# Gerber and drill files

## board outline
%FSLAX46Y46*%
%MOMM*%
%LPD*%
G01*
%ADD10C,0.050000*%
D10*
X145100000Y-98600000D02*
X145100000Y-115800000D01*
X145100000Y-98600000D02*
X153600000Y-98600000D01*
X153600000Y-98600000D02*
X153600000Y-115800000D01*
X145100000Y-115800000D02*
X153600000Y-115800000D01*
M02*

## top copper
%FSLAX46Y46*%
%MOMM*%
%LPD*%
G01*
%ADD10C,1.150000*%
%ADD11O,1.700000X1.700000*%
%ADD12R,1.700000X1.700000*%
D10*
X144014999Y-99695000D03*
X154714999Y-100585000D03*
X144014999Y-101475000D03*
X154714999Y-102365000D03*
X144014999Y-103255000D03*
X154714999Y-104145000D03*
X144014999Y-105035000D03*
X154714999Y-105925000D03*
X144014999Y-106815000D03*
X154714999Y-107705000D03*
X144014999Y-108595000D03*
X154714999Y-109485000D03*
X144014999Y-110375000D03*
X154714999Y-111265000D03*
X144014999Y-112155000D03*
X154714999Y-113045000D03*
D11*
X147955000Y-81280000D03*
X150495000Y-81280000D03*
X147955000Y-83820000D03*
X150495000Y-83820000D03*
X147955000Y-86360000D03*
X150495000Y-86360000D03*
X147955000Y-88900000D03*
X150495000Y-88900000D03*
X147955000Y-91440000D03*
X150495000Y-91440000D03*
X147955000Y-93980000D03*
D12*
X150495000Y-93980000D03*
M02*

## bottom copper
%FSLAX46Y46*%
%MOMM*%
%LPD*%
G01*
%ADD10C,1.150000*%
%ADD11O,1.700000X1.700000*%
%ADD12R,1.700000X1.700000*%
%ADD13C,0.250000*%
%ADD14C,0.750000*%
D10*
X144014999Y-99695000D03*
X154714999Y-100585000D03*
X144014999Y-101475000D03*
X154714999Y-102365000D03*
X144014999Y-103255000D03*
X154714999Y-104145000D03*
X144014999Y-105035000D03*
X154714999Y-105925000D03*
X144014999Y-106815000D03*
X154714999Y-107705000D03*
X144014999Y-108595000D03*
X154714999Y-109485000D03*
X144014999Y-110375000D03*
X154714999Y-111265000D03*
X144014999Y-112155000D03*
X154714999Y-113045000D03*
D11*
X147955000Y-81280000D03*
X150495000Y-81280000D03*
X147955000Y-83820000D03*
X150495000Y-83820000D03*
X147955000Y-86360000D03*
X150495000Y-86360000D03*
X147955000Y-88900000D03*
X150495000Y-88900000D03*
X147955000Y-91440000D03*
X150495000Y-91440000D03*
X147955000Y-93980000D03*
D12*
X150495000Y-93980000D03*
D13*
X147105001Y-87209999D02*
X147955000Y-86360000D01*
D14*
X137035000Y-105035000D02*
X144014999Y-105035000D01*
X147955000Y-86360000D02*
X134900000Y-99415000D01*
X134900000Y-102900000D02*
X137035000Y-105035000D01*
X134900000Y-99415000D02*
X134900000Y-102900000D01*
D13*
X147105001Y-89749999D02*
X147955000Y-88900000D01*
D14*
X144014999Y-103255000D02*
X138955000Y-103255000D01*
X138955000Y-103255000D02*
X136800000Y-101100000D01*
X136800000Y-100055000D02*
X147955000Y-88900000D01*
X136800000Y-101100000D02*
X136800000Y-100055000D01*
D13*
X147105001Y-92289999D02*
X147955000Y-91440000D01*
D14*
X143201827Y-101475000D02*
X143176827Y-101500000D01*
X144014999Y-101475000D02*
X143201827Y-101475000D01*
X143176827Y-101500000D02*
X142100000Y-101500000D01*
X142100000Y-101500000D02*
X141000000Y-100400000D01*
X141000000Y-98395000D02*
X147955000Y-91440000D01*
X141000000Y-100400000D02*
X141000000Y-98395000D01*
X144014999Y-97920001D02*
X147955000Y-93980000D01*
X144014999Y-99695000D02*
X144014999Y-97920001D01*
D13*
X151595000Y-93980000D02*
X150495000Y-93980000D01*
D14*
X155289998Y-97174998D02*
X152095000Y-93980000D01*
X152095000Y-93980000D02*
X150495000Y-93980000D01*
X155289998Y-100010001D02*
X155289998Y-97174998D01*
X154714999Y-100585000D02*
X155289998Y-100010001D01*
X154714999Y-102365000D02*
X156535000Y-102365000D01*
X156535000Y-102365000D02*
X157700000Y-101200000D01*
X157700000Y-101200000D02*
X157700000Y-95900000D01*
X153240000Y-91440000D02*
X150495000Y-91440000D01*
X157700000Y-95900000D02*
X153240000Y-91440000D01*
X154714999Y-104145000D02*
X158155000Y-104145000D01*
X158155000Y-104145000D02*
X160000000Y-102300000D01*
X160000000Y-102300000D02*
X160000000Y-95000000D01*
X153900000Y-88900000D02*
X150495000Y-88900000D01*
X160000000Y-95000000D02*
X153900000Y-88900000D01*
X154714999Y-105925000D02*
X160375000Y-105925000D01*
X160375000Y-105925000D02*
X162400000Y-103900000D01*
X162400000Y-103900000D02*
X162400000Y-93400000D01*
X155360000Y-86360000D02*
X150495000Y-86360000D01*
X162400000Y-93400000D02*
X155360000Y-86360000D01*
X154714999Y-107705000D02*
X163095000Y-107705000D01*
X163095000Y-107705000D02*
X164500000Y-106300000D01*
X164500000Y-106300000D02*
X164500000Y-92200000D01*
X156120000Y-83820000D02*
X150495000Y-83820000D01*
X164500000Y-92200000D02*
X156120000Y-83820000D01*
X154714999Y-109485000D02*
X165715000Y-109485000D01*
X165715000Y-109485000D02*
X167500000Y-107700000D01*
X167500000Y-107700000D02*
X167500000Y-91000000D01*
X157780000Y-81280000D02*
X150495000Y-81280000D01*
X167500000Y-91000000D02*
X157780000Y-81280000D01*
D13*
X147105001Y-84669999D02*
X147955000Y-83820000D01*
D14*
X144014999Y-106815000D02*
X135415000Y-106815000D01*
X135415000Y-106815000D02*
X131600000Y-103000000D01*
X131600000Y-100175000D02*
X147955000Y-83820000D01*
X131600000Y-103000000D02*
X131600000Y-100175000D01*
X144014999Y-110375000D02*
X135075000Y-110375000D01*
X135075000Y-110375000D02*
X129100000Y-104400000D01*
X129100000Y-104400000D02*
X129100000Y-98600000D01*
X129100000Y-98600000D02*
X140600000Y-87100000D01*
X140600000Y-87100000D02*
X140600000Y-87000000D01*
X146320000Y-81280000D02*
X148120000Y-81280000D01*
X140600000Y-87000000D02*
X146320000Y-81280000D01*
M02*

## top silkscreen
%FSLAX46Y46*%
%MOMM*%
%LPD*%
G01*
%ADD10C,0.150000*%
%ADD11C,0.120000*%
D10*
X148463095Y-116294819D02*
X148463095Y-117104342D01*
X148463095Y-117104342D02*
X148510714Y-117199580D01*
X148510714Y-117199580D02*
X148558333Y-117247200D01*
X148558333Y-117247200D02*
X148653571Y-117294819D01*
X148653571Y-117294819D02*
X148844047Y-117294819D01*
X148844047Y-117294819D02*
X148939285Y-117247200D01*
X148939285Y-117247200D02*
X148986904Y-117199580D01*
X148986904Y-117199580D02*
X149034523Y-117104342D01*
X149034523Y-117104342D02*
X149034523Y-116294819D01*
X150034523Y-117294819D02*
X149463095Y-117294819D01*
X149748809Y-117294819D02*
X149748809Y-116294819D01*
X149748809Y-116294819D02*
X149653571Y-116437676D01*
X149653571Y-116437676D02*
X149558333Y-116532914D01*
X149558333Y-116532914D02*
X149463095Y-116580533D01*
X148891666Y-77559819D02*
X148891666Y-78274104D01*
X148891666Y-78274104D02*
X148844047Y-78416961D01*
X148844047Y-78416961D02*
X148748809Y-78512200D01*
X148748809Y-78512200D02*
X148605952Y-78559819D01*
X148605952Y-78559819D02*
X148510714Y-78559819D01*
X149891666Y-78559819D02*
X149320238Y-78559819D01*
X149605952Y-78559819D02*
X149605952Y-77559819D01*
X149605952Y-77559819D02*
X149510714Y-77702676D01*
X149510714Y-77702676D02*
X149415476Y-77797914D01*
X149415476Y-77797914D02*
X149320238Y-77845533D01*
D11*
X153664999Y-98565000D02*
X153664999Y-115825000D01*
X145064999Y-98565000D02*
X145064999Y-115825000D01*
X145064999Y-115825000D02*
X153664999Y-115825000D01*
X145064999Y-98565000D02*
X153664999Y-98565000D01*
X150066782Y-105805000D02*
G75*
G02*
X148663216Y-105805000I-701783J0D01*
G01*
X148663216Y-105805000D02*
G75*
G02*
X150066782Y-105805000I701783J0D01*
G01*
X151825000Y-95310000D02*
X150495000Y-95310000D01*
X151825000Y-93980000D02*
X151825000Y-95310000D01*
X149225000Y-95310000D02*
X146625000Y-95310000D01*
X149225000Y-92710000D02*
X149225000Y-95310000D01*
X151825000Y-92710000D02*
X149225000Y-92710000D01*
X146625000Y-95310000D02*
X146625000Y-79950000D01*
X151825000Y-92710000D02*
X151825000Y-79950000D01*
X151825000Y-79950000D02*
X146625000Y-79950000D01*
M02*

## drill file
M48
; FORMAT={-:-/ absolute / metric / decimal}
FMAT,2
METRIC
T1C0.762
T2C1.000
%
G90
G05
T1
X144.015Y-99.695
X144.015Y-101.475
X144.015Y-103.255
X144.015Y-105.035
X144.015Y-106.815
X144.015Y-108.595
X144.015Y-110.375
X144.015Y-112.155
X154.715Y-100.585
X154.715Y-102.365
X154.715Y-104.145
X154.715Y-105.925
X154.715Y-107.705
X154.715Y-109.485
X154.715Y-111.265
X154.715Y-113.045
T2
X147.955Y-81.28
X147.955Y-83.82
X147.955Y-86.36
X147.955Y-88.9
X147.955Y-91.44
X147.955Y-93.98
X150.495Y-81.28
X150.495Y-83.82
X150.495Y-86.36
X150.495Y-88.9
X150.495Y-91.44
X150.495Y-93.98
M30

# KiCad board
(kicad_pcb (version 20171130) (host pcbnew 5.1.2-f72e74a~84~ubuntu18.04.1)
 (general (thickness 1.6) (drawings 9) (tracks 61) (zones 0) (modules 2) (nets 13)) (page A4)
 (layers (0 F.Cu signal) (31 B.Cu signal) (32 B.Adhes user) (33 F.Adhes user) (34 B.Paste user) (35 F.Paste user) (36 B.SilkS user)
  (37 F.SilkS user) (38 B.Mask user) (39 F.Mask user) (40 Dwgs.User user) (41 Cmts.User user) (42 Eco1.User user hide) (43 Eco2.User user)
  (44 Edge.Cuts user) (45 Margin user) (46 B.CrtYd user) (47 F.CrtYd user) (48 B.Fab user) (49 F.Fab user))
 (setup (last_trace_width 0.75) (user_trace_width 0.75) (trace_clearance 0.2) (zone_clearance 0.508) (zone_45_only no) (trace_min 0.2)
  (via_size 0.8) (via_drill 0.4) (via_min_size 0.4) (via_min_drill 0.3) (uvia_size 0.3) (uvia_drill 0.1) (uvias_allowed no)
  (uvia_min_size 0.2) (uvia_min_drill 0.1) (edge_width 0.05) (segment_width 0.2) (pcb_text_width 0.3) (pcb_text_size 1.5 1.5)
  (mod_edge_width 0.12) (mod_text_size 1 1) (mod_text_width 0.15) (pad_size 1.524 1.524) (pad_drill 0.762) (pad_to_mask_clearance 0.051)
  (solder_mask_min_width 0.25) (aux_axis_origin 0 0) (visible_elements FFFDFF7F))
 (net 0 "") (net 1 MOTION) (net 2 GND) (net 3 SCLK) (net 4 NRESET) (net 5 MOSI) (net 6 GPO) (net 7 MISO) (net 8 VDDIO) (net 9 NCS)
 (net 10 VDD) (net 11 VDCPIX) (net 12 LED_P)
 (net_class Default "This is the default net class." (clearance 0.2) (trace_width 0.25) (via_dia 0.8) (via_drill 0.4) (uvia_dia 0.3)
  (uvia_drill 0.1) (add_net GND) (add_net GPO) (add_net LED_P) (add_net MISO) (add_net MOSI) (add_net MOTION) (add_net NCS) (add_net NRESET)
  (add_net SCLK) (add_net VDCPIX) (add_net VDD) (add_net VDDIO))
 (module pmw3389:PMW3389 (layer F.Cu) (at 149.364999 105.805)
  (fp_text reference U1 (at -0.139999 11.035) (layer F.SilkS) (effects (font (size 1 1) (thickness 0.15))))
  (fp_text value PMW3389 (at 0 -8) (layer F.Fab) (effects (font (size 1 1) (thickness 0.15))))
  (fp_line (start 4.3 -7.24) (end 4.3 10.02) (layer F.SilkS) (width 0.12))
  (fp_line (start -4.3 -7.24) (end -4.3 10.02) (layer F.SilkS) (width 0.12))
  (fp_line (start -4.3 10.02) (end 4.3 10.02) (layer F.SilkS) (width 0.12))
  (fp_line (start -4.3 -7.24) (end 4.3 -7.24) (layer F.SilkS) (width 0.12))
  (fp_circle (center 0 0) (end 0.7 -0.05) (layer F.SilkS) (width 0.12))
  (pad 9 thru_hole circle (at -5.35 -6.11) (size 1.15 1.15) (drill 0.762) (layers *.Cu *.Mask) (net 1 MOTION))
  (pad 8 thru_hole circle (at 5.35 -5.22) (size 1.15 1.15) (drill 0.762) (layers *.Cu *.Mask) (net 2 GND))
  (pad 10 thru_hole circle (at -5.35 -4.33) (size 1.15 1.15) (drill 0.762) (layers *.Cu *.Mask) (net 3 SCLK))
  (pad 7 thru_hole circle (at 5.35 -3.44) (size 1.15 1.15) (drill 0.762) (layers *.Cu *.Mask) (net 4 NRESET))
  (pad 11 thru_hole circle (at -5.35 -2.55) (size 1.15 1.15) (drill 0.762) (layers *.Cu *.Mask) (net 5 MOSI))
  (pad 6 thru_hole circle (at 5.35 -1.66) (size 1.15 1.15) (drill 0.762) (layers *.Cu *.Mask) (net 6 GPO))
  (pad 12 thru_hole circle (at -5.35 -0.77) (size 1.15 1.15) (drill 0.762) (layers *.Cu *.Mask) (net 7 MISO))
  (pad 5 thru_hole circle (at 5.35 0.12) (size 1.15 1.15) (drill 0.762) (layers *.Cu *.Mask) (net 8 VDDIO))
  (pad 13 thru_hole circle (at -5.35 1.01) (size 1.15 1.15) (drill 0.762) (layers *.Cu *.Mask) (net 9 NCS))
  (pad 4 thru_hole circle (at 5.35 1.9) (size 1.15 1.15) (drill 0.762) (layers *.Cu *.Mask) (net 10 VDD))
  (pad 14 thru_hole circle (at -5.35 2.79) (size 1.15 1.15) (drill 0.762) (layers *.Cu *.Mask))
  (pad 3 thru_hole circle (at 5.35 3.68) (size 1.15 1.15) (drill 0.762) (layers *.Cu *.Mask) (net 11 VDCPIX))
  (pad 15 thru_hole circle (at -5.35 4.57) (size 1.15 1.15) (drill 0.762) (layers *.Cu *.Mask) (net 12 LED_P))
  (pad 2 thru_hole circle (at 5.35 5.46) (size 1.15 1.15) (drill 0.762) (layers *.Cu *.Mask))
  (pad 16 thru_hole circle (at -5.35 6.35) (size 1.15 1.15) (drill 0.762) (layers *.Cu *.Mask))
  (pad 1 thru_hole circle (at 5.35 7.24) (size 1.15 1.15) (drill 0.762) (layers *.Cu *.Mask)))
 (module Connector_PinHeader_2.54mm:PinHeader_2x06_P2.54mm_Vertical (layer F.Cu) (at 150.495 93.98 180)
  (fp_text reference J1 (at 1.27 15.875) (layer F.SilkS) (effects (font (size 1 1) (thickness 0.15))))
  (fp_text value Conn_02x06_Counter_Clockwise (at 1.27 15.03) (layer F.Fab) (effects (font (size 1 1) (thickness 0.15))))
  (fp_line (start -1.33 -1.33) (end 0 -1.33) (layer F.SilkS) (width 0.12))
  (fp_line (start -1.33 0) (end -1.33 -1.33) (layer F.SilkS) (width 0.12))
  (fp_line (start 1.27 -1.33) (end 3.87 -1.33) (layer F.SilkS) (width 0.12))
  (fp_line (start 1.27 1.27) (end 1.27 -1.33) (layer F.SilkS) (width 0.12))
  (fp_line (start -1.33 1.27) (end 1.27 1.27) (layer F.SilkS) (width 0.12))
  (fp_line (start 3.87 -1.33) (end 3.87 14.03) (layer F.SilkS) (width 0.12))
  (fp_line (start -1.33 1.27) (end -1.33 14.03) (layer F.SilkS) (width 0.12))
  (fp_line (start -1.33 14.03) (end 3.87 14.03) (layer F.SilkS) (width 0.12))
  (pad 12 thru_hole oval (at 2.54 12.7 180) (size 1.7 1.7) (drill 1) (layers *.Cu *.Mask) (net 12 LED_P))
  (pad 11 thru_hole oval (at 0 12.7 180) (size 1.7 1.7) (drill 1) (layers *.Cu *.Mask) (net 11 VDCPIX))
  (pad 10 thru_hole oval (at 2.54 10.16 180) (size 1.7 1.7) (drill 1) (layers *.Cu *.Mask) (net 9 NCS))
  (pad 9 thru_hole oval (at 0 10.16 180) (size 1.7 1.7) (drill 1) (layers *.Cu *.Mask) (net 10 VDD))
  (pad 8 thru_hole oval (at 2.54 7.62 180) (size 1.7 1.7) (drill 1) (layers *.Cu *.Mask) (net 7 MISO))
  (pad 7 thru_hole oval (at 0 7.62 180) (size 1.7 1.7) (drill 1) (layers *.Cu *.Mask) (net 8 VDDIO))
  (pad 6 thru_hole oval (at 2.54 5.08 180) (size 1.7 1.7) (drill 1) (layers *.Cu *.Mask) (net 5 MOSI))
  (pad 5 thru_hole oval (at 0 5.08 180) (size 1.7 1.7) (drill 1) (layers *.Cu *.Mask) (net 6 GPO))
  (pad 4 thru_hole oval (at 2.54 2.54 180) (size 1.7 1.7) (drill 1) (layers *.Cu *.Mask) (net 3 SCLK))
  (pad 3 thru_hole oval (at 0 2.54 180) (size 1.7 1.7) (drill 1) (layers *.Cu *.Mask) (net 4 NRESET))
  (pad 2 thru_hole oval (at 2.54 0 180) (size 1.7 1.7) (drill 1) (layers *.Cu *.Mask) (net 1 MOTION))
  (pad 1 thru_hole rect (at 0 0 180) (size 1.7 1.7) (drill 1) (layers *.Cu *.Mask) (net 2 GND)))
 (gr_line (start 145.1 98.6) (end 145.1 115.8) (layer Edge.Cuts) (width 0.05))
 (gr_line (start 145.1 98.6) (end 153.6 98.6) (layer Edge.Cuts) (width 0.05))
 (gr_line (start 153.6 98.6) (end 153.6 115.8) (layer Edge.Cuts) (width 0.05))
 (gr_line (start 145.1 115.8) (end 153.6 115.8) (layer Edge.Cuts) (width 0.05))
 (segment (start 147.105001 87.209999) (end 147.955 86.36) (width 0.25) (layer B.Cu) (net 7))
 (segment (start 137.035 105.035) (end 144.014999 105.035) (width 0.75) (layer B.Cu) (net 7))
 (segment (start 147.955 86.36) (end 134.9 99.415) (width 0.75) (layer B.Cu) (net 7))
 (segment (start 134.9 102.9) (end 137.035 105.035) (width 0.75) (layer B.Cu) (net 7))
 (segment (start 134.9 99.415) (end 134.9 102.9) (width 0.75) (layer B.Cu) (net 7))
 (segment (start 147.105001 89.749999) (end 147.955 88.9) (width 0.25) (layer B.Cu) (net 5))
 (segment (start 144.014999 103.255) (end 138.955 103.255) (width 0.75) (layer B.Cu) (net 5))
 (segment (start 138.955 103.255) (end 136.8 101.1) (width 0.75) (layer B.Cu) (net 5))
 (segment (start 136.8 100.055) (end 147.955 88.9) (width 0.75) (layer B.Cu) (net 5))
 (segment (start 136.8 101.1) (end 136.8 100.055) (width 0.75) (layer B.Cu) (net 5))
 (segment (start 147.105001 92.289999) (end 147.955 91.44) (width 0.25) (layer B.Cu) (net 3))
 (segment (start 143.201827 101.475) (end 143.176827 101.5) (width 0.75) (layer B.Cu) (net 3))
 (segment (start 144.014999 101.475) (end 143.201827 101.475) (width 0.75) (layer B.Cu) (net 3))
 (segment (start 143.176827 101.5) (end 142.1 101.5) (width 0.75) (layer B.Cu) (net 3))
 (segment (start 142.1 101.5) (end 141 100.4) (width 0.75) (layer B.Cu) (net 3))
 (segment (start 141 98.395) (end 147.955 91.44) (width 0.75) (layer B.Cu) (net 3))
 (segment (start 141 100.4) (end 141 98.395) (width 0.75) (layer B.Cu) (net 3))
 (segment (start 144.014999 97.920001) (end 147.955 93.98) (width 0.75) (layer B.Cu) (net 1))
 (segment (start 144.014999 99.695) (end 144.014999 97.920001) (width 0.75) (layer B.Cu) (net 1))
 (segment (start 151.595 93.98) (end 150.495 93.98) (width 0.25) (layer B.Cu) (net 2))
 (segment (start 155.289998 97.174998) (end 152.095 93.98) (width 0.75) (layer B.Cu) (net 2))
 (segment (start 152.095 93.98) (end 150.495 93.98) (width 0.75) (layer B.Cu) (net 2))
 (segment (start 155.289998 100.010001) (end 155.289998 97.174998) (width 0.75) (layer B.Cu) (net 2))
 (segment (start 154.714999 100.585) (end 155.289998 100.010001) (width 0.75) (layer B.Cu) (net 2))
 (segment (start 154.714999 102.365) (end 156.535 102.365) (width 0.75) (layer B.Cu) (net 4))
 (segment (start 156.535 102.365) (end 157.7 101.2) (width 0.75) (layer B.Cu) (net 4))
 (segment (start 157.7 101.2) (end 157.7 95.9) (width 0.75) (layer B.Cu) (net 4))
 (segment (start 153.24 91.44) (end 150.495 91.44) (width 0.75) (layer B.Cu) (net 4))
 (segment (start 157.7 95.9) (end 153.24 91.44) (width 0.75) (layer B.Cu) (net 4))
 (segment (start 154.714999 104.145) (end 158.155 104.145) (width 0.75) (layer B.Cu) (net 6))
 (segment (start 158.155 104.145) (end 160 102.3) (width 0.75) (layer B.Cu) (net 6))
 (segment (start 160 102.3) (end 160 95) (width 0.75) (layer B.Cu) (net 6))
 (segment (start 153.9 88.9) (end 150.495 88.9) (width 0.75) (layer B.Cu) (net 6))
 (segment (start 160 95) (end 153.9 88.9) (width 0.75) (layer B.Cu) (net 6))
 (segment (start 154.714999 105.925) (end 160.375 105.925) (width 0.75) (layer B.Cu) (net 8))
 (segment (start 160.375 105.925) (end 162.4 103.9) (width 0.75) (layer B.Cu) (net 8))
 (segment (start 162.4 103.9) (end 162.4 93.4) (width 0.75) (layer B.Cu) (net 8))
 (segment (start 155.36 86.36) (end 150.495 86.36) (width 0.75) (layer B.Cu) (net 8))
 (segment (start 162.4 93.4) (end 155.36 86.36) (width 0.75) (layer B.Cu) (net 8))
 (segment (start 154.714999 107.705) (end 163.095 107.705) (width 0.75) (layer B.Cu) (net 10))
 (segment (start 163.095 107.705) (end 164.5 106.3) (width 0.75) (layer B.Cu) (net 10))
 (segment (start 164.5 106.3) (end 164.5 92.2) (width 0.75) (layer B.Cu) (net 10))
 (segment (start 156.12 83.82) (end 150.495 83.82) (width 0.75) (layer B.Cu) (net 10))
 (segment (start 164.5 92.2) (end 156.12 83.82) (width 0.75) (layer B.Cu) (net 10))
 (segment (start 154.714999 109.485) (end 165.715 109.485) (width 0.75) (layer B.Cu) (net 11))
 (segment (start 165.715 109.485) (end 167.5 107.7) (width 0.75) (layer B.Cu) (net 11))
 (segment (start 167.5 107.7) (end 167.5 91) (width 0.75) (layer B.Cu) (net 11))
 (segment (start 157.78 81.28) (end 150.495 81.28) (width 0.75) (layer B.Cu) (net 11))
 (segment (start 167.5 91) (end 157.78 81.28) (width 0.75) (layer B.Cu) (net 11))
 (segment (start 147.105001 84.669999) (end 147.955 83.82) (width 0.25) (layer B.Cu) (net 9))
 (segment (start 144.014999 106.815) (end 135.415 106.815) (width 0.75) (layer B.Cu) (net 9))
 (segment (start 135.415 106.815) (end 131.6 103) (width 0.75) (layer B.Cu) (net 9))
 (segment (start 131.6 100.175) (end 147.955 83.82) (width 0.75) (layer B.Cu) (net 9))
 (segment (start 131.6 103) (end 131.6 100.175) (width 0.75) (layer B.Cu) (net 9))
 (segment (start 144.014999 110.375) (end 135.075 110.375) (width 0.75) (layer B.Cu) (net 12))
 (segment (start 135.075 110.375) (end 129.1 104.4) (width 0.75) (layer B.Cu) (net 12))
 (segment (start 129.1 104.4) (end 129.1 98.6) (width 0.75) (layer B.Cu) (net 12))
 (segment (start 129.1 98.6) (end 140.6 87.1) (width 0.75) (layer B.Cu) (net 12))
 (segment (start 140.6 87.1) (end 140.6 87) (width 0.75) (layer B.Cu) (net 12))
 (segment (start 146.32 81.28) (end 148.12 81.28) (width 0.75) (layer B.Cu) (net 12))
 (segment (start 140.6 87) (end 146.32 81.28) (width 0.75) (layer B.Cu) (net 12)))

